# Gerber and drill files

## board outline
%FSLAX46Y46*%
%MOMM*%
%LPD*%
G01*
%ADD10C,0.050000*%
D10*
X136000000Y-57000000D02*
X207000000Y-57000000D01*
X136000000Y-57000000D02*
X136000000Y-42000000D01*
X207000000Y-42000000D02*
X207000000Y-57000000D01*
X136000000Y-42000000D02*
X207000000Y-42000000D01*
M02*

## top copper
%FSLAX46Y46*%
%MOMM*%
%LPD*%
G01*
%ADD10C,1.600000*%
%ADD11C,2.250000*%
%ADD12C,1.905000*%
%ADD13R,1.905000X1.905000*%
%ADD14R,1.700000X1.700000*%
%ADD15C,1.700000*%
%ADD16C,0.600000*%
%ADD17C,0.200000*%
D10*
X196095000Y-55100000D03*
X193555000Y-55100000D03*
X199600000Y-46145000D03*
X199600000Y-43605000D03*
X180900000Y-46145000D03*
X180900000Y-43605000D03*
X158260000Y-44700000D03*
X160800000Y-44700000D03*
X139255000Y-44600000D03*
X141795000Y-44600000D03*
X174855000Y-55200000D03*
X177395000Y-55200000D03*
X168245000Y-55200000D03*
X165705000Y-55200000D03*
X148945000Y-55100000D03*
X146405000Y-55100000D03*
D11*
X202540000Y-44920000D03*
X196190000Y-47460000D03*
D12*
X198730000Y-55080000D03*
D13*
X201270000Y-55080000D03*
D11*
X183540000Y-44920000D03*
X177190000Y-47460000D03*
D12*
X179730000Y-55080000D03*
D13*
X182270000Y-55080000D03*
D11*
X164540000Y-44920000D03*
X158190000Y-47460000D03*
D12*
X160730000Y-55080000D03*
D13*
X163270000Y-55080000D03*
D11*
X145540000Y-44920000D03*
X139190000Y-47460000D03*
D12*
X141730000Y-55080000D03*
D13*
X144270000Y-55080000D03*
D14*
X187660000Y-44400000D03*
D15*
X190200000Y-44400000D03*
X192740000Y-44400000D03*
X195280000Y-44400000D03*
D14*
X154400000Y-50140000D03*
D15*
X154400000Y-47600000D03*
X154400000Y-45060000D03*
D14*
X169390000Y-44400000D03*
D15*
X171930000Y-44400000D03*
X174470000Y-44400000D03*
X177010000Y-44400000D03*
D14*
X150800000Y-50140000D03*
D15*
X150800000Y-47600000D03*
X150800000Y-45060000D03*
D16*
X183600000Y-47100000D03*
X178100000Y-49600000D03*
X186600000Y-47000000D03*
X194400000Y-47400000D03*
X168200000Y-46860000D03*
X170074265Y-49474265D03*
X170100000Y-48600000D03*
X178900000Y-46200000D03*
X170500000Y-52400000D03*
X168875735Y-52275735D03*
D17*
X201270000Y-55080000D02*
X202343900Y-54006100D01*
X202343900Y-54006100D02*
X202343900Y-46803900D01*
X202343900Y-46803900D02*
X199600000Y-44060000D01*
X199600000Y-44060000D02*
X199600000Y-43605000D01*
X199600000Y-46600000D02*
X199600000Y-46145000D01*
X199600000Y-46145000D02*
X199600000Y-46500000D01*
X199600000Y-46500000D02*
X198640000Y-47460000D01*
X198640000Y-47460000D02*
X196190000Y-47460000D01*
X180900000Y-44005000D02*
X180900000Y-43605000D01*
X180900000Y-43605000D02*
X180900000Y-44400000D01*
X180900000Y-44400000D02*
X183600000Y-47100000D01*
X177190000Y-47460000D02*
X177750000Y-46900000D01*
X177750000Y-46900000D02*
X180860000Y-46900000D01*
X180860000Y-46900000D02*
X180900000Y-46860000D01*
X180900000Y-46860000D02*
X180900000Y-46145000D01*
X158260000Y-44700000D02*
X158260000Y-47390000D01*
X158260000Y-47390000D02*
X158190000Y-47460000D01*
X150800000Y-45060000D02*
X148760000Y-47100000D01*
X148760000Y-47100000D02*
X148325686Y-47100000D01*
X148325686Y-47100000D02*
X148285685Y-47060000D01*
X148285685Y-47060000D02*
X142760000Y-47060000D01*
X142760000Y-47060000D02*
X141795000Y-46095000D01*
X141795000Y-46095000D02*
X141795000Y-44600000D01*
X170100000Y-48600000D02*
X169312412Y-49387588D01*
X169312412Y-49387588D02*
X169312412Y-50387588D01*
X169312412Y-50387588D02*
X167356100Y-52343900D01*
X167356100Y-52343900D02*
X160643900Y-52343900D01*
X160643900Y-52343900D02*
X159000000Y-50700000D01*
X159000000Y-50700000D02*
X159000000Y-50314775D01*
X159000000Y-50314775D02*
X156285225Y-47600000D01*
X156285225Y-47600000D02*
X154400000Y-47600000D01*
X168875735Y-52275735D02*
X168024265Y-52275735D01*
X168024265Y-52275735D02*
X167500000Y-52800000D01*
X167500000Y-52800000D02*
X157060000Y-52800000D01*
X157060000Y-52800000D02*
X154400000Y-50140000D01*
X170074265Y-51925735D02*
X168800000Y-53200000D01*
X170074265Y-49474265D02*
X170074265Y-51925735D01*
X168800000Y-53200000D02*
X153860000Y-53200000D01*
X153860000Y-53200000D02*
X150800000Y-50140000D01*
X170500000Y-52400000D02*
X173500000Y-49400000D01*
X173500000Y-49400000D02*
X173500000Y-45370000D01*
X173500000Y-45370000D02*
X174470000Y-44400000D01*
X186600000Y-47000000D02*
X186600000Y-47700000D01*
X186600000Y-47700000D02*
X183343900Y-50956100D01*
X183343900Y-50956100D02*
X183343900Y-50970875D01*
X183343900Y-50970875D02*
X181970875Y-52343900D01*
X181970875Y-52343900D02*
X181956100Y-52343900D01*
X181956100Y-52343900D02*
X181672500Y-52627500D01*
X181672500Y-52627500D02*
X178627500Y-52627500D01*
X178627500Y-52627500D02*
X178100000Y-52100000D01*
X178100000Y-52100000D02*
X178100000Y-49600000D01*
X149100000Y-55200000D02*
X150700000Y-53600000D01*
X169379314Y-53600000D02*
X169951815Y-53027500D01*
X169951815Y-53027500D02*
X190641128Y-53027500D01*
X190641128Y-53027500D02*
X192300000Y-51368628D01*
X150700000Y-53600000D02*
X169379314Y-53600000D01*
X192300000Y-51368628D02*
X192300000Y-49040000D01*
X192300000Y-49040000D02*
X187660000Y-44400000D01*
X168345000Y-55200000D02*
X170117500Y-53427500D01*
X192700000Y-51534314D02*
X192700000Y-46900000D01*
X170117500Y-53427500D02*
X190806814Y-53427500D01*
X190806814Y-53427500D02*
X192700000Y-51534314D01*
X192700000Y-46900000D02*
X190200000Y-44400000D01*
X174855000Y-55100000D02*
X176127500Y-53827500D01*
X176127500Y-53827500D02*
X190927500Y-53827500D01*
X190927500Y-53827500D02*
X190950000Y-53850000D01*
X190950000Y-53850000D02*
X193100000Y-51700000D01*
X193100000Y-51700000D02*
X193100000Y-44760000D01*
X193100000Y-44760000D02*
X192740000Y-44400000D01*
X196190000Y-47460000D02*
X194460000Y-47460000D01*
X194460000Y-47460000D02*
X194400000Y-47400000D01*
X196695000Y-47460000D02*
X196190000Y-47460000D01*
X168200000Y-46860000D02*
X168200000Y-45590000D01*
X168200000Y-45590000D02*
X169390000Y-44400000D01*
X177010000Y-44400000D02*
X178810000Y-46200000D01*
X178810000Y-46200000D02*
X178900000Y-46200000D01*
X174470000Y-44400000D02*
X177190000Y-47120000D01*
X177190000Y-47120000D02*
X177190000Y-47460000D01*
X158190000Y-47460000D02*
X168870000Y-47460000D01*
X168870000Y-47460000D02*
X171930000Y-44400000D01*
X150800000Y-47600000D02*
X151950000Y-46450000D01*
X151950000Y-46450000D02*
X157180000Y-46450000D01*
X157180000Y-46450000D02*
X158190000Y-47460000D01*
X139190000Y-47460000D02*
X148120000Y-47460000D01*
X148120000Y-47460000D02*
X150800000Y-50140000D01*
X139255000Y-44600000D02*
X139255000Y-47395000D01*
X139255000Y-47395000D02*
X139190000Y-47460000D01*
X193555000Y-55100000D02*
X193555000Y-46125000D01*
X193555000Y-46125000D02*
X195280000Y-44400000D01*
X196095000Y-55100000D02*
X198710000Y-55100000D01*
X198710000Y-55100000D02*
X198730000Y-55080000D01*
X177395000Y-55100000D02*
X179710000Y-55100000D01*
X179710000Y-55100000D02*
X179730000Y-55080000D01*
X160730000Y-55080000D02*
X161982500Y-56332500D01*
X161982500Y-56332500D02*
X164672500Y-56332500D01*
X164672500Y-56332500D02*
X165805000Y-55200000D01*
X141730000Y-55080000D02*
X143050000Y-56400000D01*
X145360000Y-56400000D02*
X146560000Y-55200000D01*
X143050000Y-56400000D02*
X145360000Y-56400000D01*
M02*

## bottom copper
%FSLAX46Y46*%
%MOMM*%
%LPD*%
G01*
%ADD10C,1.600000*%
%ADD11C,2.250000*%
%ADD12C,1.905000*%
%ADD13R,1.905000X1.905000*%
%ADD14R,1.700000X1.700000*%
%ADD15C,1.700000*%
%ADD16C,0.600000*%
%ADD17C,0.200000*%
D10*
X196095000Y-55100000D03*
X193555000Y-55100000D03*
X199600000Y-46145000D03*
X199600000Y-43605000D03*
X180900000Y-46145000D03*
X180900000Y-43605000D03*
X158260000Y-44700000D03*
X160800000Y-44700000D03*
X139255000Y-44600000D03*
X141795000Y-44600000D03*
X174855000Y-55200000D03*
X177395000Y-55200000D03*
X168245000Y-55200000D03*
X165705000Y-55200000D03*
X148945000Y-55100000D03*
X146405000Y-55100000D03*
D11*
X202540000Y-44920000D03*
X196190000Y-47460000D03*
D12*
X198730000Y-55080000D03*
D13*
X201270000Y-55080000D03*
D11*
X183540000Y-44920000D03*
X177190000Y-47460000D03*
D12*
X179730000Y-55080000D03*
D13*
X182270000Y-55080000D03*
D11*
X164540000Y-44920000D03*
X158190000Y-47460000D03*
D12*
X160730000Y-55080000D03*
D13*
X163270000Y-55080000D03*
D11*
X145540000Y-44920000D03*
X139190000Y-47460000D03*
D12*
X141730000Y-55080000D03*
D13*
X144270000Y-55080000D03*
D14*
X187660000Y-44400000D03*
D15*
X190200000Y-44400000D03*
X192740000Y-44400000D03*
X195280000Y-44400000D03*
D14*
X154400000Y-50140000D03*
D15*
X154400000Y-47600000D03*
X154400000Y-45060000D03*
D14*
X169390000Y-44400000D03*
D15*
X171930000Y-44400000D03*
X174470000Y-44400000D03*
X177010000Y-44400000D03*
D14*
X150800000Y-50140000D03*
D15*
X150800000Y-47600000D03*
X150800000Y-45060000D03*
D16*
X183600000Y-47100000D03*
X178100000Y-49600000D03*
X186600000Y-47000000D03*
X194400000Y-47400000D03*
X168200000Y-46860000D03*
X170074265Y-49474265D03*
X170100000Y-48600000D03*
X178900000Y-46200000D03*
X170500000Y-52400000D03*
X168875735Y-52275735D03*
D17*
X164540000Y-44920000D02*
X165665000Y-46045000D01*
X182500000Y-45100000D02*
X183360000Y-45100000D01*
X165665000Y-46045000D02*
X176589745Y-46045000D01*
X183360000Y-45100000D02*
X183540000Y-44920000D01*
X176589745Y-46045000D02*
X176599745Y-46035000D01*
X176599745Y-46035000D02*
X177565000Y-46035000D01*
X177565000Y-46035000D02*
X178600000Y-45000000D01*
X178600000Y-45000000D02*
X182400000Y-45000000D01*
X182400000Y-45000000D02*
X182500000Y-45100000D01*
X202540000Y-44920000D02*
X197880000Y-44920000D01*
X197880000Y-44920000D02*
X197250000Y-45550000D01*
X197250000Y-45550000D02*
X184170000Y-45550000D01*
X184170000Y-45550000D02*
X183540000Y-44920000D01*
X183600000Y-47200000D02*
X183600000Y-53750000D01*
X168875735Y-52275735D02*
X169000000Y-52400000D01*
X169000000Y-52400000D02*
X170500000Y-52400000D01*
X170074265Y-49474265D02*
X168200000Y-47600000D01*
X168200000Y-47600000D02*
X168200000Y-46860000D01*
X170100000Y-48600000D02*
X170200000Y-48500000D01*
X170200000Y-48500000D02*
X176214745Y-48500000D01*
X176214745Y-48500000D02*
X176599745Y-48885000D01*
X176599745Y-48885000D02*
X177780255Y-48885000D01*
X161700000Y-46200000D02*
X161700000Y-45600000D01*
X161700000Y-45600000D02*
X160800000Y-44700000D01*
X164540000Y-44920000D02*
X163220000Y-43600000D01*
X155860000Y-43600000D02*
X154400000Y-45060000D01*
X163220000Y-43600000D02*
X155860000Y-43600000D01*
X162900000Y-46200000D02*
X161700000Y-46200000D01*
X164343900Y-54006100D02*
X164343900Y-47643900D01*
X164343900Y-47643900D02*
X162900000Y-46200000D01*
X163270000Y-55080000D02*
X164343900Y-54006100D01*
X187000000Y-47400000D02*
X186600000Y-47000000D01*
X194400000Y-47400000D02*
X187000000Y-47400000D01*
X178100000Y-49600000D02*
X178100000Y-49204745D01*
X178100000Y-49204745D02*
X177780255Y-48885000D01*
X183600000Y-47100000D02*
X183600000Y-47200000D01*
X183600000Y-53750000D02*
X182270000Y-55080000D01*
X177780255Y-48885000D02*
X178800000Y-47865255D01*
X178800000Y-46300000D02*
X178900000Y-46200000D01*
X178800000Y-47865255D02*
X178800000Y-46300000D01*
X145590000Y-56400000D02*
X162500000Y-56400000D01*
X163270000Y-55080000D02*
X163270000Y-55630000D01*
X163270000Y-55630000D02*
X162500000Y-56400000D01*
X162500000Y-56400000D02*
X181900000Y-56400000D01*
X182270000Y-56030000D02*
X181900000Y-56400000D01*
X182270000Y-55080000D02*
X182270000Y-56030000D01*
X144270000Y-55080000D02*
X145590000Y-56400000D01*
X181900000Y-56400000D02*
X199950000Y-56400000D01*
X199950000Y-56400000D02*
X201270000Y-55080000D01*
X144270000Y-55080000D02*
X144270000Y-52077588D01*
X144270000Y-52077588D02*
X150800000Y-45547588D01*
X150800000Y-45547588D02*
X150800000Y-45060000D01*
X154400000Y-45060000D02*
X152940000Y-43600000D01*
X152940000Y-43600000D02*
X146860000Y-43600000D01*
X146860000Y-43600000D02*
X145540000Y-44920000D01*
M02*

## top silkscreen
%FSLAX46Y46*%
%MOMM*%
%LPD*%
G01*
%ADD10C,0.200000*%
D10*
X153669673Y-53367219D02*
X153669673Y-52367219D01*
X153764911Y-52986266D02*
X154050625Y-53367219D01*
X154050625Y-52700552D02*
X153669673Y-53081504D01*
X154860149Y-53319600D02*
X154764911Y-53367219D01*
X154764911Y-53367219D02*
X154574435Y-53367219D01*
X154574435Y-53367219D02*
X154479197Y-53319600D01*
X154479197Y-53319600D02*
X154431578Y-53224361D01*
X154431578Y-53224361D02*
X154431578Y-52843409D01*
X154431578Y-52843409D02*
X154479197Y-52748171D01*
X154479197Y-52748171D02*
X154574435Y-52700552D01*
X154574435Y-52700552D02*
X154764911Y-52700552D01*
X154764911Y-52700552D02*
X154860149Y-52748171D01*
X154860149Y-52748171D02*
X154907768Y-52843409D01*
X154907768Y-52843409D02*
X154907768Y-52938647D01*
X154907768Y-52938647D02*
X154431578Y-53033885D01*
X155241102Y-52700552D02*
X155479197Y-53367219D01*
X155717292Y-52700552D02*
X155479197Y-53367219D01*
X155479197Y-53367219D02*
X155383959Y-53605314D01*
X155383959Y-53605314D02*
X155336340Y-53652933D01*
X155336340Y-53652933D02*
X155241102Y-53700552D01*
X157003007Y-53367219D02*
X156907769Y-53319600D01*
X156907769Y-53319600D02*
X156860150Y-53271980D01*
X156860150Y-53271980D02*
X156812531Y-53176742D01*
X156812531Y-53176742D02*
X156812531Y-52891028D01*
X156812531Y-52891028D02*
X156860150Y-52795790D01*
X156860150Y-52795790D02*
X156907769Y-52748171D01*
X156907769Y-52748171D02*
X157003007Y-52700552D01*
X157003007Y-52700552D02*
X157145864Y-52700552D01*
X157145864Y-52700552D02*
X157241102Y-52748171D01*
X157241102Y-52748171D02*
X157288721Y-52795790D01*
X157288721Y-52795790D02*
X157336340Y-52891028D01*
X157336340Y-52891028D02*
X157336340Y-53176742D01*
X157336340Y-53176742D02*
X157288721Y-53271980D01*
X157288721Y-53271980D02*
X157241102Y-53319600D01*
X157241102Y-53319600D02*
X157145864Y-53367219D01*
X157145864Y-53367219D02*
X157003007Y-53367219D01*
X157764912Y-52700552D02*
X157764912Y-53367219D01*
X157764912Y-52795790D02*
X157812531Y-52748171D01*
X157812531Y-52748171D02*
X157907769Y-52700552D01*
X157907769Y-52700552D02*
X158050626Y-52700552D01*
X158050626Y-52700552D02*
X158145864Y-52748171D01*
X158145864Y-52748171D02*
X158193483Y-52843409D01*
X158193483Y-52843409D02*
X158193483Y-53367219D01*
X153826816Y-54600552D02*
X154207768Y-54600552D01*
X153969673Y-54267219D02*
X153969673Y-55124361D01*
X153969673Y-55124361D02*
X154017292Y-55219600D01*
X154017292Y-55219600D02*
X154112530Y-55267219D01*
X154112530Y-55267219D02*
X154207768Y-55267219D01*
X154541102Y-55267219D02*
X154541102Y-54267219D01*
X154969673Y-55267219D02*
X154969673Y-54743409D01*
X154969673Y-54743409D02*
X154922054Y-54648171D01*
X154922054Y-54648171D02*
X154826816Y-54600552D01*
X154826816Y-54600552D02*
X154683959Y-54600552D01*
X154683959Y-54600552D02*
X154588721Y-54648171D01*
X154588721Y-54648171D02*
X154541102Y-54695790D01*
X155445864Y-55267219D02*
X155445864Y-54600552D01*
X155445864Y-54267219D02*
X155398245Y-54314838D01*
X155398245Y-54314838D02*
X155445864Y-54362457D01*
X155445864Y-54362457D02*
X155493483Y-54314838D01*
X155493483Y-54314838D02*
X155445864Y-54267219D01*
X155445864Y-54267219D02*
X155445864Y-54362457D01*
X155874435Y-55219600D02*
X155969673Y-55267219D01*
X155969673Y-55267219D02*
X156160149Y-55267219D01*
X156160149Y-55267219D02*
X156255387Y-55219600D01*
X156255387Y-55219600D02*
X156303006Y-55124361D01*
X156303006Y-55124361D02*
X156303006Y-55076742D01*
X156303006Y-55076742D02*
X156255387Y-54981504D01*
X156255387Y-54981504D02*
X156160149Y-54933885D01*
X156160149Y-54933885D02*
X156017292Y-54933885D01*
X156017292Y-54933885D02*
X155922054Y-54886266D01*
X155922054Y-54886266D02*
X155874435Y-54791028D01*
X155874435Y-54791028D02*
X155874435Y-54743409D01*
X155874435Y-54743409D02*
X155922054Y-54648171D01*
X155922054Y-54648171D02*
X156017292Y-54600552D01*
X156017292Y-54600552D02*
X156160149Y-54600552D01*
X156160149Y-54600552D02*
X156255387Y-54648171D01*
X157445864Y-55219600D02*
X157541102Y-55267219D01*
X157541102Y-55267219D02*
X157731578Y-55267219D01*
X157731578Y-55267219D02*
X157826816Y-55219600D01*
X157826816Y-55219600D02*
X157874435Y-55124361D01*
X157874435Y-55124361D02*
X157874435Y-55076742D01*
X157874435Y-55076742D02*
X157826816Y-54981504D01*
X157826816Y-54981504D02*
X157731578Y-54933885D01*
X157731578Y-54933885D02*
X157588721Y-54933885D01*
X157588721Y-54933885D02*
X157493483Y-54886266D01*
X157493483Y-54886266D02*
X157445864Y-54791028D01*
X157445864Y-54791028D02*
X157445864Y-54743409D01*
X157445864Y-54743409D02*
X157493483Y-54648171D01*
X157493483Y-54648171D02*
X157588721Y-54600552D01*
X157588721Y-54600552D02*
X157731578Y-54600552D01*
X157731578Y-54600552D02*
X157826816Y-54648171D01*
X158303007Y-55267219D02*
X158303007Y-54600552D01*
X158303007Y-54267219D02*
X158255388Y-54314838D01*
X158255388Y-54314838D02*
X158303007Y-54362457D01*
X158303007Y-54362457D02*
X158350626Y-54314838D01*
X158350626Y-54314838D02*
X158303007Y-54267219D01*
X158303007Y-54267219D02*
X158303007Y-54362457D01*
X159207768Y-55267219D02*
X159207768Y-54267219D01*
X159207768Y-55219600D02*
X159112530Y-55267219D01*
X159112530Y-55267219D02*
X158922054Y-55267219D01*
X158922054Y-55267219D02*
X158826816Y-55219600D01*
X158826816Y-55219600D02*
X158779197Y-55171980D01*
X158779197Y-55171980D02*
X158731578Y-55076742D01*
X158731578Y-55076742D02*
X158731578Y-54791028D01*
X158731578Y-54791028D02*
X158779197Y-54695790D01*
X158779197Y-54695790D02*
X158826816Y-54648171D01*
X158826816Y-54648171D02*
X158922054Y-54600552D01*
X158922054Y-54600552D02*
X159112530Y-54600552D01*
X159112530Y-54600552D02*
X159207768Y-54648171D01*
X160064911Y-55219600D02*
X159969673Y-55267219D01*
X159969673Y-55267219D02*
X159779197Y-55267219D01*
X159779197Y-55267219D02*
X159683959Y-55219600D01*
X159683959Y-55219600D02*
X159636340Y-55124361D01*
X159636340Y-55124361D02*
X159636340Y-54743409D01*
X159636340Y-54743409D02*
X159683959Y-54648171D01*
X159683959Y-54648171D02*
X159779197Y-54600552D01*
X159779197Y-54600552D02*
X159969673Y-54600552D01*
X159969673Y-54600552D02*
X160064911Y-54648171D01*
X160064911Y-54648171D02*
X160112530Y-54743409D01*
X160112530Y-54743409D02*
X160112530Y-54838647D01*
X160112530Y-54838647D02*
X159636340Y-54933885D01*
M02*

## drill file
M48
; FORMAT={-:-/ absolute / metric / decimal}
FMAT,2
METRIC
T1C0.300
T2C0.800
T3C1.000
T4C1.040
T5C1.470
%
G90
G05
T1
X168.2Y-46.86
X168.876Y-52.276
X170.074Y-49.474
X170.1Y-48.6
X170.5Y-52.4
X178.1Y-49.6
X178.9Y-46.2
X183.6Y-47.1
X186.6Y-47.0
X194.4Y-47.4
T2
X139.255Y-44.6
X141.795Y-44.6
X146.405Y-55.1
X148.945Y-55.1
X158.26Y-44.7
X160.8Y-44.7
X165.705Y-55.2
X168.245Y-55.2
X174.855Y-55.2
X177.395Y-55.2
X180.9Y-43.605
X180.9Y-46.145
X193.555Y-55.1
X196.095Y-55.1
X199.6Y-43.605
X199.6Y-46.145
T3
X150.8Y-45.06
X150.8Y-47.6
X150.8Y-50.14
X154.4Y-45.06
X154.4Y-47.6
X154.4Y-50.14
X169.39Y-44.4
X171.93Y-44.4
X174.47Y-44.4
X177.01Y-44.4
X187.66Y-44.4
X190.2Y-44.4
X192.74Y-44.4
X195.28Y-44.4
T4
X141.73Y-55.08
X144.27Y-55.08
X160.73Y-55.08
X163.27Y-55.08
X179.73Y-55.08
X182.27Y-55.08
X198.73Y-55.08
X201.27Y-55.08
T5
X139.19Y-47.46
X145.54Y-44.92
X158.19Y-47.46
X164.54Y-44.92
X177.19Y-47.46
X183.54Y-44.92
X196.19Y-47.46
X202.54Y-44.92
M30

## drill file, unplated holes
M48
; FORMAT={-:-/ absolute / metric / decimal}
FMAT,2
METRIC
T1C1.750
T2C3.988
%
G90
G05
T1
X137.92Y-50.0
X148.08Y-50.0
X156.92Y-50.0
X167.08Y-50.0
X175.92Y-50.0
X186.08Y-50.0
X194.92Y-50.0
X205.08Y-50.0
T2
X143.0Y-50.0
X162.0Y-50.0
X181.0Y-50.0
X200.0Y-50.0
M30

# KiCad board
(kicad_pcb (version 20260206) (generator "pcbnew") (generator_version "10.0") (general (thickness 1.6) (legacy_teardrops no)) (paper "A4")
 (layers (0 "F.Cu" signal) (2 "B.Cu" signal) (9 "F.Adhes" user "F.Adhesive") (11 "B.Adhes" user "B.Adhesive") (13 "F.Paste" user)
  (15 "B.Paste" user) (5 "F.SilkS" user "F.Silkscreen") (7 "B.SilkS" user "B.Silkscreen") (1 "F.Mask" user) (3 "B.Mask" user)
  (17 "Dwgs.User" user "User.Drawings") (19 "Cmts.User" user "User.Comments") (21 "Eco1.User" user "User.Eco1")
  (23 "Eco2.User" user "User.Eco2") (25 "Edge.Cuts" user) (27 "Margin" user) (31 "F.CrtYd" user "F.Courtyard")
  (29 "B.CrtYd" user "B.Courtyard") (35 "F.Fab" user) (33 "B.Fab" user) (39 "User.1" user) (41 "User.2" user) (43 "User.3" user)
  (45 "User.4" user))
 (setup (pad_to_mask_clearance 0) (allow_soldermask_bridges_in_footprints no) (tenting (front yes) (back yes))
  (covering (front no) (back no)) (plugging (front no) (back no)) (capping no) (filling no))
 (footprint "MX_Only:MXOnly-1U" (layer "F.Cu") (at 200 50)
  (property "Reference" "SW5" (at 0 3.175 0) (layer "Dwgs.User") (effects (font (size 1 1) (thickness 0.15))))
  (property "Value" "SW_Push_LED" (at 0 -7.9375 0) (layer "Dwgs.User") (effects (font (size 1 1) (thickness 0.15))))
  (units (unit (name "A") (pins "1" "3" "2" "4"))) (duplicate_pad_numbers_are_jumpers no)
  (pad "" np_thru_hole circle (at -5.08 0 48.0996) (size 1.75 1.75) (drill 1.75) (layers "*.Cu" "*.Mask"))
  (pad "" np_thru_hole circle (at 0 0) (size 3.9878 3.9878) (drill 3.9878) (layers "*.Cu" "*.Mask"))
  (pad "" np_thru_hole circle (at 5.08 0 48.0996) (size 1.75 1.75) (drill 1.75) (layers "*.Cu" "*.Mask"))
  (pad "1" thru_hole circle (at -3.81 -2.54) (size 2.25 2.25) (drill 1.47) (layers "*.Cu" "B.Mask") (remove_unused_layers no) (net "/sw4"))
  (pad "2" thru_hole circle (at 2.54 -5.08) (size 2.25 2.25) (drill 1.47) (layers "*.Cu" "B.Mask") (remove_unused_layers no) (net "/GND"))
  (pad "3" thru_hole circle (at -1.27 5.08) (size 1.905 1.905) (drill 1.04) (layers "*.Cu" "B.Mask") (remove_unused_layers no)
   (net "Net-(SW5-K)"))
  (pad "4" thru_hole rect (at 1.27 5.08) (size 1.905 1.905) (drill 1.04) (layers "*.Cu" "B.Mask") (remove_unused_layers no) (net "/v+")))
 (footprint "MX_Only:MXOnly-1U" (layer "F.Cu") (at 162 50)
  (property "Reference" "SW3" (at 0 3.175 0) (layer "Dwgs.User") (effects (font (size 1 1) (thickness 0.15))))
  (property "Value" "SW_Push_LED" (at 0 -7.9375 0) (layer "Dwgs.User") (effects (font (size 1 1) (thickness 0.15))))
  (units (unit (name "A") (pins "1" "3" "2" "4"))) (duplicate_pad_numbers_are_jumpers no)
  (pad "" np_thru_hole circle (at -5.08 0 48.0996) (size 1.75 1.75) (drill 1.75) (layers "*.Cu" "*.Mask"))
  (pad "" np_thru_hole circle (at 0 0) (size 3.9878 3.9878) (drill 3.9878) (layers "*.Cu" "*.Mask"))
  (pad "" np_thru_hole circle (at 5.08 0 48.0996) (size 1.75 1.75) (drill 1.75) (layers "*.Cu" "*.Mask"))
  (pad "1" thru_hole circle (at -3.81 -2.54) (size 2.25 2.25) (drill 1.47) (layers "*.Cu" "B.Mask") (remove_unused_layers no) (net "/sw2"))
  (pad "2" thru_hole circle (at 2.54 -5.08) (size 2.25 2.25) (drill 1.47) (layers "*.Cu" "B.Mask") (remove_unused_layers no) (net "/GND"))
  (pad "3" thru_hole circle (at -1.27 5.08) (size 1.905 1.905) (drill 1.04) (layers "*.Cu" "B.Mask") (remove_unused_layers no)
   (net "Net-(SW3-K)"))
  (pad "4" thru_hole rect (at 1.27 5.08) (size 1.905 1.905) (drill 1.04) (layers "*.Cu" "B.Mask") (remove_unused_layers no) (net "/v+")))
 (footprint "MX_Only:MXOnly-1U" (layer "F.Cu") (at 181 50)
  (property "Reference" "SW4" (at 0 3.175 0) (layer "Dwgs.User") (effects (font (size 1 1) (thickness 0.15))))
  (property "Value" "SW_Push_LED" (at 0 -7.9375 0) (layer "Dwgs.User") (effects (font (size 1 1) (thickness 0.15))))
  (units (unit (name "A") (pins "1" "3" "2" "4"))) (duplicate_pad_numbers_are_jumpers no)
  (pad "" np_thru_hole circle (at -5.08 0 48.0996) (size 1.75 1.75) (drill 1.75) (layers "*.Cu" "*.Mask"))
  (pad "" np_thru_hole circle (at 0 0) (size 3.9878 3.9878) (drill 3.9878) (layers "*.Cu" "*.Mask"))
  (pad "" np_thru_hole circle (at 5.08 0 48.0996) (size 1.75 1.75) (drill 1.75) (layers "*.Cu" "*.Mask"))
  (pad "1" thru_hole circle (at -3.81 -2.54) (size 2.25 2.25) (drill 1.47) (layers "*.Cu" "B.Mask") (remove_unused_layers no) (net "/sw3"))
  (pad "2" thru_hole circle (at 2.54 -5.08) (size 2.25 2.25) (drill 1.47) (layers "*.Cu" "B.Mask") (remove_unused_layers no) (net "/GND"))
  (pad "3" thru_hole circle (at -1.27 5.08) (size 1.905 1.905) (drill 1.04) (layers "*.Cu" "B.Mask") (remove_unused_layers no)
   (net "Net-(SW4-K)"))
  (pad "4" thru_hole rect (at 1.27 5.08) (size 1.905 1.905) (drill 1.04) (layers "*.Cu" "B.Mask") (remove_unused_layers no) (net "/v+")))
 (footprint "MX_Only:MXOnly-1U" (layer "F.Cu") (at 143 50)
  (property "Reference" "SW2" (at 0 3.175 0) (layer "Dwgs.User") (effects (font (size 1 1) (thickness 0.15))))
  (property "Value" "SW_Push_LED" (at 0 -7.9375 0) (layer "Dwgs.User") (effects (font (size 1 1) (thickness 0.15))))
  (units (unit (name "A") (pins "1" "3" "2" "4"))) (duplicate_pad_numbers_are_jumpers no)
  (pad "" np_thru_hole circle (at -5.08 0 48.0996) (size 1.75 1.75) (drill 1.75) (layers "*.Cu" "*.Mask"))
  (pad "" np_thru_hole circle (at 0 0) (size 3.9878 3.9878) (drill 3.9878) (layers "*.Cu" "*.Mask"))
  (pad "" np_thru_hole circle (at 5.08 0 48.0996) (size 1.75 1.75) (drill 1.75) (layers "*.Cu" "*.Mask"))
  (pad "1" thru_hole circle (at -3.81 -2.54) (size 2.25 2.25) (drill 1.47) (layers "*.Cu" "B.Mask") (remove_unused_layers no) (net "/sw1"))
  (pad "2" thru_hole circle (at 2.54 -5.08) (size 2.25 2.25) (drill 1.47) (layers "*.Cu" "B.Mask") (remove_unused_layers no) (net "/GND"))
  (pad "3" thru_hole circle (at -1.27 5.08) (size 1.905 1.905) (drill 1.04) (layers "*.Cu" "B.Mask") (remove_unused_layers no)
   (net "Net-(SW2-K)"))
  (pad "4" thru_hole rect (at 1.27 5.08) (size 1.905 1.905) (drill 1.04) (layers "*.Cu" "B.Mask") (remove_unused_layers no) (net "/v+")))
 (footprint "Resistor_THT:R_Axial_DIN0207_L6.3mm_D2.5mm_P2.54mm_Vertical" (layer "B.Cu") (at 174.855 55.2)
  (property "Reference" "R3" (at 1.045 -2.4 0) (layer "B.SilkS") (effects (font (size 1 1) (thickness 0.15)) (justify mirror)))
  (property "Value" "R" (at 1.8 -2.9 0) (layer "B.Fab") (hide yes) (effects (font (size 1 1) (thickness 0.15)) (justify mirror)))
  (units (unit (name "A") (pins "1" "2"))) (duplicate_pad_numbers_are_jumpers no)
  (pad "1" thru_hole circle (at 0 0) (size 1.6 1.6) (drill 0.8) (layers "*.Cu" "*.Mask") (remove_unused_layers no) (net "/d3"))
  (pad "2" thru_hole circle (at 2.54 0) (size 1.6 1.6) (drill 0.8) (layers "*.Cu" "*.Mask") (remove_unused_layers no) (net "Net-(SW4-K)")))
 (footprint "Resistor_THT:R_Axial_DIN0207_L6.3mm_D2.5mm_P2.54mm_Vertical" (layer "B.Cu") (at 193.555 55.1)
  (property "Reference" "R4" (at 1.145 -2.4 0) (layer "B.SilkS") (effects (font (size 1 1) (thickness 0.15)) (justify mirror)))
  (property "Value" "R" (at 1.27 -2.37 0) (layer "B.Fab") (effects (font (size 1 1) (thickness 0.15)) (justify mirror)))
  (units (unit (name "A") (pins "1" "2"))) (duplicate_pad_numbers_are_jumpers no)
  (pad "1" thru_hole circle (at 0 0) (size 1.6 1.6) (drill 0.8) (layers "*.Cu" "*.Mask") (remove_unused_layers no) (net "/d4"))
  (pad "2" thru_hole circle (at 2.54 0) (size 1.6 1.6) (drill 0.8) (layers "*.Cu" "*.Mask") (remove_unused_layers no) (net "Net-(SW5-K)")))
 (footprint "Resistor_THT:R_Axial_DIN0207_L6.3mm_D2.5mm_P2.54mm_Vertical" (layer "B.Cu") (at 158.26 44.7)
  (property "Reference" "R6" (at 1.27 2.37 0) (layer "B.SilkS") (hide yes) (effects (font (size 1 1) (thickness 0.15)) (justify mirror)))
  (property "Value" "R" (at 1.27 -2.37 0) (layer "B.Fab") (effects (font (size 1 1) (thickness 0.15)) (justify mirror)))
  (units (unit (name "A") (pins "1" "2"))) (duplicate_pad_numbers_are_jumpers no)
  (pad "1" thru_hole circle (at 0 0) (size 1.6 1.6) (drill 0.8) (layers "*.Cu" "*.Mask") (remove_unused_layers no) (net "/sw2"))
  (pad "2" thru_hole circle (at 2.54 0) (size 1.6 1.6) (drill 0.8) (layers "*.Cu" "*.Mask") (remove_unused_layers no) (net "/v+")))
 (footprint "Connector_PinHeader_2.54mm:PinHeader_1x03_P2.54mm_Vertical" (layer "B.Cu") (at 154.4 50.14)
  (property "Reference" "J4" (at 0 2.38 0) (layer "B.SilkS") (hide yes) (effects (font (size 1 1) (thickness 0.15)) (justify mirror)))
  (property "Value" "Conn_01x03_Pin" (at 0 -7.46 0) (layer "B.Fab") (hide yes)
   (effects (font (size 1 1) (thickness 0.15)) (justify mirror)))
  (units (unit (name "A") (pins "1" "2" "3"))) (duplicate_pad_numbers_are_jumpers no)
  (pad "1" thru_hole rect (at 0 0) (size 1.7 1.7) (drill 1) (layers "*.Cu" "*.Mask") (remove_unused_layers no) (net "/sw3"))
  (pad "2" thru_hole circle (at 0 -2.54) (size 1.7 1.7) (drill 1) (layers "*.Cu" "*.Mask") (remove_unused_layers no) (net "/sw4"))
  (pad "3" thru_hole circle (at 0 -5.08) (size 1.7 1.7) (drill 1) (layers "*.Cu" "*.Mask") (remove_unused_layers no) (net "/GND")))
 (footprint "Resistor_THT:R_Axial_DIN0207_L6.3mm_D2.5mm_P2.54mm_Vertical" (layer "B.Cu") (at 168.245 55.2 180)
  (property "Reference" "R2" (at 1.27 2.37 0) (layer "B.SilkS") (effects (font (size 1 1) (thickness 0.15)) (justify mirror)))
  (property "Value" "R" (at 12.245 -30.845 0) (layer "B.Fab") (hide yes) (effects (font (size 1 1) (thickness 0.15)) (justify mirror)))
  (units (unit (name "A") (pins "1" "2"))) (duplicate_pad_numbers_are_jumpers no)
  (pad "1" thru_hole circle (at 0 0 180) (size 1.6 1.6) (drill 0.8) (layers "*.Cu" "*.Mask") (remove_unused_layers no) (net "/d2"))
  (pad "2" thru_hole circle (at 2.54 0 180) (size 1.6 1.6) (drill 0.8) (layers "*.Cu" "*.Mask") (remove_unused_layers no)
   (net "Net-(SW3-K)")))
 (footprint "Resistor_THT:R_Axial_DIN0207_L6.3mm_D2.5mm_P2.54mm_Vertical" (layer "B.Cu") (at 180.9 46.145 90)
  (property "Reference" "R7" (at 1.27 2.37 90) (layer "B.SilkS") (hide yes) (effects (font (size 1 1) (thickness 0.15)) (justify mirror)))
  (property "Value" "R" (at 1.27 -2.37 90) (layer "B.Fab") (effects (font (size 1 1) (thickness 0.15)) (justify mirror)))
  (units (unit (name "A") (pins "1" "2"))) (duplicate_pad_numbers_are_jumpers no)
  (pad "1" thru_hole circle (at 0 0 90) (size 1.6 1.6) (drill 0.8) (layers "*.Cu" "*.Mask") (remove_unused_layers no) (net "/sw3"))
  (pad "2" thru_hole circle (at 2.54 0 90) (size 1.6 1.6) (drill 0.8) (layers "*.Cu" "*.Mask") (remove_unused_layers no) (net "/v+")))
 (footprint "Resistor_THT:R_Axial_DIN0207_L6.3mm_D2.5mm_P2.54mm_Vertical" (layer "B.Cu") (at 148.945 55.1 180)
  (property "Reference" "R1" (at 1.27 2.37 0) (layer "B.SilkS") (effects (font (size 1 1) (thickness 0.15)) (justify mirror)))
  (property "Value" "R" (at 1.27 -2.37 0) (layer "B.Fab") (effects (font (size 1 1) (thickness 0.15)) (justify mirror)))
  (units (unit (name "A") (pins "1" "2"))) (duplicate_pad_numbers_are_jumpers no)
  (pad "1" thru_hole circle (at 0 0 180) (size 1.6 1.6) (drill 0.8) (layers "*.Cu" "*.Mask") (remove_unused_layers no) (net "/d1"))
  (pad "2" thru_hole circle (at 2.54 0 180) (size 1.6 1.6) (drill 0.8) (layers "*.Cu" "*.Mask") (remove_unused_layers no)
   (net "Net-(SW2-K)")))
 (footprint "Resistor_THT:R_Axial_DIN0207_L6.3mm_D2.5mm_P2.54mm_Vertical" (layer "B.Cu") (at 139.255 44.6)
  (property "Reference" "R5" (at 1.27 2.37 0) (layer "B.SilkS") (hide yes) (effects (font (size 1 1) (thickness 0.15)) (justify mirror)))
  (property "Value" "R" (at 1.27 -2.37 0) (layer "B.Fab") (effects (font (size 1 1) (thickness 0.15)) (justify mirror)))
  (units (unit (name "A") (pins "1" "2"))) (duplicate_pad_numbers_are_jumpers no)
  (pad "1" thru_hole circle (at 0 0) (size 1.6 1.6) (drill 0.8) (layers "*.Cu" "*.Mask") (remove_unused_layers no) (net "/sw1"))
  (pad "2" thru_hole circle (at 2.54 0) (size 1.6 1.6) (drill 0.8) (layers "*.Cu" "*.Mask") (remove_unused_layers no) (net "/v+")))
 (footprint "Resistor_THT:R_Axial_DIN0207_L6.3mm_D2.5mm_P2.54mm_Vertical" (layer "B.Cu") (at 199.6 46.145 90)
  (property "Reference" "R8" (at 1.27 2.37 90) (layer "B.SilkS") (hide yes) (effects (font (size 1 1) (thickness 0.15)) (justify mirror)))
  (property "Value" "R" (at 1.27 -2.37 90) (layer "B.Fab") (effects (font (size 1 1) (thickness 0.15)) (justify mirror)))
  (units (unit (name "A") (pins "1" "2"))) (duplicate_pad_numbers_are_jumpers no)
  (pad "1" thru_hole circle (at 0 0 90) (size 1.6 1.6) (drill 0.8) (layers "*.Cu" "*.Mask") (remove_unused_layers no) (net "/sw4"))
  (pad "2" thru_hole circle (at 2.54 0 90) (size 1.6 1.6) (drill 0.8) (layers "*.Cu" "*.Mask") (remove_unused_layers no) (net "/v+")))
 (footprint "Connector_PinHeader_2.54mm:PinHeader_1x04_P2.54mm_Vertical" (layer "B.Cu") (at 169.39 44.4 -90)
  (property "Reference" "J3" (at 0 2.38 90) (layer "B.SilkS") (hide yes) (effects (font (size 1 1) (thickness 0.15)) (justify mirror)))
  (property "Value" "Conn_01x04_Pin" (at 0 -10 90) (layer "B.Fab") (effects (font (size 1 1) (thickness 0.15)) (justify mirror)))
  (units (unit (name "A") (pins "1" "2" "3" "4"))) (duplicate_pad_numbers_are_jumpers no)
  (pad "1" thru_hole rect (at 0 0 270) (size 1.7 1.7) (drill 1) (layers "*.Cu" "*.Mask") (remove_unused_layers no) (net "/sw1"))
  (pad "2" thru_hole circle (at 0 -2.54 270) (size 1.7 1.7) (drill 1) (layers "*.Cu" "*.Mask") (remove_unused_layers no) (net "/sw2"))
  (pad "3" thru_hole circle (at 0 -5.08 270) (size 1.7 1.7) (drill 1) (layers "*.Cu" "*.Mask") (remove_unused_layers no) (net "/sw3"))
  (pad "4" thru_hole circle (at 0 -7.62 270) (size 1.7 1.7) (drill 1) (layers "*.Cu" "*.Mask") (remove_unused_layers no) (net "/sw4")))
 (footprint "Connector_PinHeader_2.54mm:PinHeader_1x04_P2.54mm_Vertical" (layer "B.Cu") (at 187.66 44.4 -90)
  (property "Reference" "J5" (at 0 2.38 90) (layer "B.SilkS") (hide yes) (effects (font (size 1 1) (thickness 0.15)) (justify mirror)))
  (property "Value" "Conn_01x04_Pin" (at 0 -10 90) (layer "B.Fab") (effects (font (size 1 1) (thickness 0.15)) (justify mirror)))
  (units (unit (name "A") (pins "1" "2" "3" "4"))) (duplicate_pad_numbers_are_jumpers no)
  (pad "1" thru_hole rect (at 0 0 270) (size 1.7 1.7) (drill 1) (layers "*.Cu" "*.Mask") (remove_unused_layers no) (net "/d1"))
  (pad "2" thru_hole circle (at 0 -2.54 270) (size 1.7 1.7) (drill 1) (layers "*.Cu" "*.Mask") (remove_unused_layers no) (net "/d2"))
  (pad "3" thru_hole circle (at 0 -5.08 270) (size 1.7 1.7) (drill 1) (layers "*.Cu" "*.Mask") (remove_unused_layers no) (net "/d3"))
  (pad "4" thru_hole circle (at 0 -7.62 270) (size 1.7 1.7) (drill 1) (layers "*.Cu" "*.Mask") (remove_unused_layers no) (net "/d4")))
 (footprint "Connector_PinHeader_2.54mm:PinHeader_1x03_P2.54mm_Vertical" (layer "B.Cu") (at 150.8 50.14)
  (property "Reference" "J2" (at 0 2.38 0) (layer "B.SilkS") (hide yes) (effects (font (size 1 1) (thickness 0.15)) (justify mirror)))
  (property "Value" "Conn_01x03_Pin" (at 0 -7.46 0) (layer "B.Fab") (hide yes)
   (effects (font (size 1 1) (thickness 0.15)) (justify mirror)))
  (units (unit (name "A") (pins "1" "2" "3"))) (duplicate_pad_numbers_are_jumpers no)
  (pad "1" thru_hole rect (at 0 0) (size 1.7 1.7) (drill 1) (layers "*.Cu" "*.Mask") (remove_unused_layers no) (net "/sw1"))
  (pad "2" thru_hole circle (at 0 -2.54) (size 1.7 1.7) (drill 1) (layers "*.Cu" "*.Mask") (remove_unused_layers no) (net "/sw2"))
  (pad "3" thru_hole circle (at 0 -5.08) (size 1.7 1.7) (drill 1) (layers "*.Cu" "*.Mask") (remove_unused_layers no) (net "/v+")))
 (gr_line (start 136 42) (end 207 42) (stroke (width 0.05) (type solid)) (layer "Edge.Cuts"))
 (gr_line (start 136 57) (end 136 42) (stroke (width 0.05) (type default)) (layer "Edge.Cuts"))
 (gr_line (start 136 57) (end 207 57) (stroke (width 0.05) (type solid)) (layer "Edge.Cuts"))
 (gr_line (start 207 42) (end 207 57) (stroke (width 0.05) (type solid)) (layer "Edge.Cuts"))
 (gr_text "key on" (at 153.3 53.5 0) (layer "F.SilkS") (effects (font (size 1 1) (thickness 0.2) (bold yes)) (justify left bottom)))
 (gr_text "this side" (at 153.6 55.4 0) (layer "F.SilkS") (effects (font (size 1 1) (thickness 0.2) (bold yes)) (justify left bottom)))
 (segment (start 199.6 44.06) (end 199.6 43.605) (width 0.2) (layer "F.Cu") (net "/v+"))
 (segment (start 201.27 55.08) (end 202.3439 54.0061) (width 0.2) (layer "F.Cu") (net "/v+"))
 (segment (start 150.8 45.06) (end 148.76 47.1) (width 0.2) (layer "F.Cu") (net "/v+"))
 (segment (start 180.9 44.005) (end 180.9 43.605) (width 0.2) (layer "F.Cu") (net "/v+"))
 (segment (start 148.76 47.1) (end 148.325686 47.1) (width 0.2) (layer "F.Cu") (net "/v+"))
 (segment (start 142.76 47.06) (end 141.795 46.095) (width 0.2) (layer "F.Cu") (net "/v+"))
 (segment (start 148.325686 47.1) (end 148.285685 47.06) (width 0.2) (layer "F.Cu") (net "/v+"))
 (segment (start 202.3439 54.0061) (end 202.3439 46.8039) (width 0.2) (layer "F.Cu") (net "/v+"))
 (segment (start 180.9 44.4) (end 183.6 47.1) (width 0.2) (layer "F.Cu") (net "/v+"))
 (segment (start 141.795 46.095) (end 141.795 44.6) (width 0.2) (layer "F.Cu") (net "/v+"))
 (segment (start 148.285685 47.06) (end 142.76 47.06) (width 0.2) (layer "F.Cu") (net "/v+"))
 (segment (start 180.9 43.605) (end 180.9 44.4) (width 0.2) (layer "F.Cu") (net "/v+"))
 (segment (start 202.3439 46.8039) (end 199.6 44.06) (width 0.2) (layer "F.Cu") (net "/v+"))
 (via (at 183.6 47.1) (size 0.6) (drill 0.3) (layers "F.Cu" "B.Cu") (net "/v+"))
 (segment (start 163.27 55.63) (end 162.5 56.4) (width 0.2) (layer "B.Cu") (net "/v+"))
 (segment (start 163.27 55.08) (end 164.3439 54.0061) (width 0.2) (layer "B.Cu") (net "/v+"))
 (segment (start 144.27 52.077588) (end 150.8 45.547588) (width 0.2) (layer "B.Cu") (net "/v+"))
 (segment (start 150.8 45.547588) (end 150.8 45.06) (width 0.2) (layer "B.Cu") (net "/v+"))
 (segment (start 161.7 45.6) (end 160.8 44.7) (width 0.2) (layer "B.Cu") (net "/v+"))
 (segment (start 199.95 56.4) (end 201.27 55.08) (width 0.2) (layer "B.Cu") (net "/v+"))
 (segment (start 161.7 46.2) (end 161.7 45.6) (width 0.2) (layer "B.Cu") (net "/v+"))
 (segment (start 183.6 53.75) (end 182.27 55.08) (width 0.2) (layer "B.Cu") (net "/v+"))
 (segment (start 182.27 55.08) (end 182.27 56.03) (width 0.2) (layer "B.Cu") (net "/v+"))
 (segment (start 183.6 47.2) (end 183.6 53.75) (width 0.2) (layer "B.Cu") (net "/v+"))
 (segment (start 144.27 55.08) (end 144.27 52.077588) (width 0.2) (layer "B.Cu") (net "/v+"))
 (segment (start 163.27 55.08) (end 163.27 55.63) (width 0.2) (layer "B.Cu") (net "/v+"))
 (segment (start 144.27 55.08) (end 145.59 56.4) (width 0.2) (layer "B.Cu") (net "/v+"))
 (segment (start 181.9 56.4) (end 199.95 56.4) (width 0.2) (layer "B.Cu") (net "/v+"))
 (segment (start 164.3439 54.0061) (end 164.3439 47.6439) (width 0.2) (layer "B.Cu") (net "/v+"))
 (segment (start 162.9 46.2) (end 161.7 46.2) (width 0.2) (layer "B.Cu") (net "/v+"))
 (segment (start 182.27 56.03) (end 181.9 56.4) (width 0.2) (layer "B.Cu") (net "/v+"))
 (segment (start 164.3439 47.6439) (end 162.9 46.2) (width 0.2) (layer "B.Cu") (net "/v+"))
 (segment (start 162.5 56.4) (end 181.9 56.4) (width 0.2) (layer "B.Cu") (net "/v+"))
 (segment (start 145.59 56.4) (end 162.5 56.4) (width 0.2) (layer "B.Cu") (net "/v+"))
 (segment (start 183.6 47.1) (end 183.6 47.2) (width 0.2) (layer "B.Cu") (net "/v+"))
 (segment (start 149.1 55.2) (end 150.7 53.6) (width 0.2) (layer "F.Cu") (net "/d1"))
 (segment (start 192.3 51.368628) (end 192.3 49.04) (width 0.2) (layer "F.Cu") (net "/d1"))
 (segment (start 192.3 49.04) (end 187.66 44.4) (width 0.2) (layer "F.Cu") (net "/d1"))
 (segment (start 169.951815 53.0275) (end 190.641128 53.0275) (width 0.2) (layer "F.Cu") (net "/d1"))
 (segment (start 190.641128 53.0275) (end 192.3 51.368628) (width 0.2) (layer "F.Cu") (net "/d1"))
 (segment (start 150.7 53.6) (end 169.379314 53.6) (width 0.2) (layer "F.Cu") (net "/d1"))
 (segment (start 169.379314 53.6) (end 169.951815 53.0275) (width 0.2) (layer "F.Cu") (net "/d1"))
 (segment (start 192.7 51.534314) (end 192.7 46.9) (width 0.2) (layer "F.Cu") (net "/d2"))
 (segment (start 170.1175 53.4275) (end 190.806814 53.4275) (width 0.2) (layer "F.Cu") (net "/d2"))
 (segment (start 192.7 46.9) (end 190.2 44.4) (width 0.2) (layer "F.Cu") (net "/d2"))
 (segment (start 190.806814 53.4275) (end 192.7 51.534314) (width 0.2) (layer "F.Cu") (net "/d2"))
 (segment (start 168.345 55.2) (end 170.1175 53.4275) (width 0.2) (layer "F.Cu") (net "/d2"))
 (segment (start 153.86 53.2) (end 150.8 50.14) (width 0.2) (layer "F.Cu") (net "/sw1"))
 (segment (start 168.2 45.59) (end 169.39 44.4) (width 0.2) (layer "F.Cu") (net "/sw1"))
 (segment (start 139.19 47.46) (end 148.12 47.46) (width 0.2) (layer "F.Cu") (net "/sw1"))
 (segment (start 170.074265 51.925735) (end 168.8 53.2) (width 0.2) (layer "F.Cu") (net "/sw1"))
 (segment (start 139.255 47.395) (end 139.19 47.46) (width 0.2) (layer "F.Cu") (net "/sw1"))
 (segment (start 168.2 46.86) (end 168.2 45.59) (width 0.2) (layer "F.Cu") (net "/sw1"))
 (segment (start 139.255 44.6) (end 139.255 47.395) (width 0.2) (layer "F.Cu") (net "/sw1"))
 (segment (start 170.074265 49.474265) (end 170.074265 51.925735) (width 0.2) (layer "F.Cu") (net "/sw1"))
 (segment (start 168.8 53.2) (end 153.86 53.2) (width 0.2) (layer "F.Cu") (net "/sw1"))
 (segment (start 148.12 47.46) (end 150.8 50.14) (width 0.2) (layer "F.Cu") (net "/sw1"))
 (via (at 168.2 46.86) (size 0.6) (drill 0.3) (layers "F.Cu" "B.Cu") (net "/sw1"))
 (via (at 170.074265 49.474265) (size 0.6) (drill 0.3) (layers "F.Cu" "B.Cu") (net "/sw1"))
 (segment (start 168.2 47.6) (end 168.2 46.86) (width 0.2) (layer "B.Cu") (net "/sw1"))
 (segment (start 170.074265 49.474265) (end 168.2 47.6) (width 0.2) (layer "B.Cu") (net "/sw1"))
 (segment (start 193.555 55.1) (end 193.555 46.125) (width 0.2) (layer "F.Cu") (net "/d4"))
 (segment (start 193.555 46.125) (end 195.28 44.4) (width 0.2) (layer "F.Cu") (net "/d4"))
 (segment (start 190.95 53.85) (end 193.1 51.7) (width 0.2) (layer "F.Cu") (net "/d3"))
 (segment (start 193.1 51.7) (end 193.1 44.76) (width 0.2) (layer "F.Cu") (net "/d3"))
 (segment (start 174.855 55.1) (end 176.1275 53.8275) (width 0.2) (layer "F.Cu") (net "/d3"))
 (segment (start 176.1275 53.8275) (end 190.9275 53.8275) (width 0.2) (layer "F.Cu") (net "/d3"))
 (segment (start 190.9275 53.8275) (end 190.95 53.85) (width 0.2) (layer "F.Cu") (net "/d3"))
 (segment (start 193.1 44.76) (end 192.74 44.4) (width 0.2) (layer "F.Cu") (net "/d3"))
 (segment (start 182.5 45.1) (end 183.36 45.1) (width 0.2) (layer "B.Cu") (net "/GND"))
 (segment (start 183.36 45.1) (end 183.54 44.92) (width 0.2) (layer "B.Cu") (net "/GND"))
 (segment (start 163.22 43.6) (end 155.86 43.6) (width 0.2) (layer "B.Cu") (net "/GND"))
 (segment (start 165.665 46.045) (end 176.589745 46.045) (width 0.2) (layer "B.Cu") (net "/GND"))
 (segment (start 197.25 45.55) (end 184.17 45.55) (width 0.2) (layer "B.Cu") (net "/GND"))
 (segment (start 184.17 45.55) (end 183.54 44.92) (width 0.2) (layer "B.Cu") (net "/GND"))
 (segment (start 178.6 45) (end 182.4 45) (width 0.2) (layer "B.Cu") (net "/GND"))
 (segment (start 146.86 43.6) (end 145.54 44.92) (width 0.2) (layer "B.Cu") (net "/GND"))
 (segment (start 154.4 45.06) (end 152.94 43.6) (width 0.2) (layer "B.Cu") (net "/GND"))
 (segment (start 177.565 46.035) (end 178.6 45) (width 0.2) (layer "B.Cu") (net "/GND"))
 (segment (start 164.54 44.92) (end 165.665 46.045) (width 0.2) (layer "B.Cu") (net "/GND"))
 (segment (start 176.589745 46.045) (end 176.599745 46.035) (width 0.2) (layer "B.Cu") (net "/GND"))
 (segment (start 164.54 44.92) (end 163.22 43.6) (width 0.2) (layer "B.Cu") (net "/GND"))
 (segment (start 202.54 44.92) (end 197.88 44.92) (width 0.2) (layer "B.Cu") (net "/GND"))
 (segment (start 155.86 43.6) (end 154.4 45.06) (width 0.2) (layer "B.Cu") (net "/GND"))
 (segment (start 152.94 43.6) (end 146.86 43.6) (width 0.2) (layer "B.Cu") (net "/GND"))
 (segment (start 182.4 45) (end 182.5 45.1) (width 0.2) (layer "B.Cu") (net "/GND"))
 (segment (start 197.88 44.92) (end 197.25 45.55) (width 0.2) (layer "B.Cu") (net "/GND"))
 (segment (start 176.599745 46.035) (end 177.565 46.035) (width 0.2) (layer "B.Cu") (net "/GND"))
 (segment (start 143.05 56.4) (end 145.36 56.4) (width 0.2) (layer "F.Cu") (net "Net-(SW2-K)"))
 (segment (start 145.36 56.4) (end 146.56 55.2) (width 0.2) (layer "F.Cu") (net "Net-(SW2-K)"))
 (segment (start 141.73 55.08) (end 143.05 56.4) (width 0.2) (layer "F.Cu") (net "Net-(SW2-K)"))
 (segment (start 164.6725 56.3325) (end 165.805 55.2) (width 0.2) (layer "F.Cu") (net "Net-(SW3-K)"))
 (segment (start 161.9825 56.3325) (end 164.6725 56.3325) (width 0.2) (layer "F.Cu") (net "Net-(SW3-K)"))
 (segment (start 160.73 55.08) (end 161.9825 56.3325) (width 0.2) (layer "F.Cu") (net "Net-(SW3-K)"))
 (segment (start 179.71 55.1) (end 179.73 55.08) (width 0.2) (layer "F.Cu") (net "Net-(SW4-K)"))
 (segment (start 177.395 55.1) (end 179.71 55.1) (width 0.2) (layer "F.Cu") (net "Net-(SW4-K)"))
 (segment (start 198.71 55.1) (end 198.73 55.08) (width 0.2) (layer "F.Cu") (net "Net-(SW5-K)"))
 (segment (start 196.095 55.1) (end 198.71 55.1) (width 0.2) (layer "F.Cu") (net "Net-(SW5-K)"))
 (segment (start 157.18 46.45) (end 158.19 47.46) (width 0.2) (layer "F.Cu") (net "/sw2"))
 (segment (start 158.19 47.46) (end 168.87 47.46) (width 0.2) (layer "F.Cu") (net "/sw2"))
 (segment (start 150.8 47.6) (end 151.95 46.45) (width 0.2) (layer "F.Cu") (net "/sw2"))
 (segment (start 168.87 47.46) (end 171.93 44.4) (width 0.2) (layer "F.Cu") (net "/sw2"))
 (segment (start 151.95 46.45) (end 157.18 46.45) (width 0.2) (layer "F.Cu") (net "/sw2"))
 (segment (start 158.26 47.39) (end 158.19 47.46) (width 0.2) (layer "F.Cu") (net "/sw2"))
 (segment (start 158.26 44.7) (end 158.26 47.39) (width 0.2) (layer "F.Cu") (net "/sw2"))
 (segment (start 170.5 52.4) (end 173.5 49.4) (width 0.2) (layer "F.Cu") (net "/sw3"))
 (segment (start 177.19 47.12) (end 177.19 47.46) (width 0.2) (layer "F.Cu") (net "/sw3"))
 (segment (start 167.5 52.8) (end 157.06 52.8) (width 0.2) (layer "F.Cu") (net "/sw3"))
 (segment (start 168.024265 52.275735) (end 167.5 52.8) (width 0.2) (layer "F.Cu") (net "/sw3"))
 (segment (start 177.19 47.46) (end 177.75 46.9) (width 0.2) (layer "F.Cu") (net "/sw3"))
 (segment (start 174.47 44.4) (end 177.19 47.12) (width 0.2) (layer "F.Cu") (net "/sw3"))
 (segment (start 173.5 49.4) (end 173.5 45.37) (width 0.2) (layer "F.Cu") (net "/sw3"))
 (segment (start 168.875735 52.275735) (end 168.024265 52.275735) (width 0.2) (layer "F.Cu") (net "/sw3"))
 (segment (start 180.86 46.9) (end 180.9 46.86) (width 0.2) (layer "F.Cu") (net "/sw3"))
 (segment (start 157.06 52.8) (end 154.4 50.14) (width 0.2) (layer "F.Cu") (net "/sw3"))
 (segment (start 173.5 45.37) (end 174.47 44.4) (width 0.2) (layer "F.Cu") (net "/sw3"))
 (segment (start 180.9 46.86) (end 180.9 46.145) (width 0.2) (layer "F.Cu") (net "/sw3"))
 (segment (start 177.75 46.9) (end 180.86 46.9) (width 0.2) (layer "F.Cu") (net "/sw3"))
 (via (at 168.875735 52.275735) (size 0.6) (drill 0.3) (layers "F.Cu" "B.Cu") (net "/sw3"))
 (via (at 170.5 52.4) (size 0.6) (drill 0.3) (layers "F.Cu" "B.Cu") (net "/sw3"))
 (segment (start 168.875735 52.275735) (end 169 52.4) (width 0.2) (layer "B.Cu") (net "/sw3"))
 (segment (start 169 52.4) (end 170.5 52.4) (width 0.2) (layer "B.Cu") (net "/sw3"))
 (segment (start 199.6 46.5) (end 198.64 47.46) (width 0.2) (layer "F.Cu") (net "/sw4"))
 (segment (start 199.6 46.145) (end 199.6 46.5) (width 0.2) (layer "F.Cu") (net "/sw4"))
 (segment (start 159 50.7) (end 159 50.314775) (width 0.2) (layer "F.Cu") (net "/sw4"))
 (segment (start 183.3439 50.9561) (end 183.3439 50.970875) (width 0.2) (layer "F.Cu") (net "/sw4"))
 (segment (start 196.695 47.46) (end 196.19 47.46) (width 0.2) (layer "F.Cu") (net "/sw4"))
 (segment (start 159 50.314775) (end 156.285225 47.6) (width 0.2) (layer "F.Cu") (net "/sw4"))
 (segment (start 181.970875 52.3439) (end 181.9561 52.3439) (width 0.2) (layer "F.Cu") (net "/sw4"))
 (segment (start 160.6439 52.3439) (end 159 50.7) (width 0.2) (layer "F.Cu") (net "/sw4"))
 (segment (start 178.1 52.1) (end 178.1 49.6) (width 0.2) (layer "F.Cu") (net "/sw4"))
 (segment (start 178.81 46.2) (end 178.9 46.2) (width 0.2) (layer "F.Cu") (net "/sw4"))
 (segment (start 183.3439 50.970875) (end 181.970875 52.3439) (width 0.2) (layer "F.Cu") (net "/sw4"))
 (segment (start 156.285225 47.6) (end 154.4 47.6) (width 0.2) (layer "F.Cu") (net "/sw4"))
 (segment (start 198.64 47.46) (end 196.19 47.46) (width 0.2) (layer "F.Cu") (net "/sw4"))
 (segment (start 199.6 46.6) (end 199.6 46.145) (width 0.2) (layer "F.Cu") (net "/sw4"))
 (segment (start 169.312412 49.387588) (end 169.312412 50.387588) (width 0.2) (layer "F.Cu") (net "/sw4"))
 (segment (start 170.1 48.6) (end 169.312412 49.387588) (width 0.2) (layer "F.Cu") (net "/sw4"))
 (segment (start 167.3561 52.3439) (end 160.6439 52.3439) (width 0.2) (layer "F.Cu") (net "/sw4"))
 (segment (start 177.01 44.4) (end 178.81 46.2) (width 0.2) (layer "F.Cu") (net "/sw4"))
 (segment (start 181.6725 52.6275) (end 178.6275 52.6275) (width 0.2) (layer "F.Cu") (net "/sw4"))
 (segment (start 169.312412 50.387588) (end 167.3561 52.3439) (width 0.2) (layer "F.Cu") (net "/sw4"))
 (segment (start 194.46 47.46) (end 194.4 47.4) (width 0.2) (layer "F.Cu") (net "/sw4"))
 (segment (start 178.6275 52.6275) (end 178.1 52.1) (width 0.2) (layer "F.Cu") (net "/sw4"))
 (segment (start 196.19 47.46) (end 194.46 47.46) (width 0.2) (layer "F.Cu") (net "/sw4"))
 (segment (start 186.6 47.7) (end 183.3439 50.9561) (width 0.2) (layer "F.Cu") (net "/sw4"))
 (segment (start 181.9561 52.3439) (end 181.6725 52.6275) (width 0.2) (layer "F.Cu") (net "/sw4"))
 (segment (start 186.6 47) (end 186.6 47.7) (width 0.2) (layer "F.Cu") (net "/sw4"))
 (via (at 170.1 48.6) (size 0.6) (drill 0.3) (layers "F.Cu" "B.Cu") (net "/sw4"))
 (via (at 194.4 47.4) (size 0.6) (drill 0.3) (layers "F.Cu" "B.Cu") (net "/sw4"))
 (via (at 178.9 46.2) (size 0.6) (drill 0.3) (layers "F.Cu" "B.Cu") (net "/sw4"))
 (via (at 186.6 47) (size 0.6) (drill 0.3) (layers "F.Cu" "B.Cu") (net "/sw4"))
 (via (at 178.1 49.6) (size 0.6) (drill 0.3) (layers "F.Cu" "B.Cu") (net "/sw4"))
 (segment (start 178.8 47.865255) (end 178.8 46.3) (width 0.2) (layer "B.Cu") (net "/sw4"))
 (segment (start 176.599745 48.885) (end 177.780255 48.885) (width 0.2) (layer "B.Cu") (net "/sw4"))
 (segment (start 176.214745 48.5) (end 176.599745 48.885) (width 0.2) (layer "B.Cu") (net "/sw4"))
 (segment (start 178.8 46.3) (end 178.9 46.2) (width 0.2) (layer "B.Cu") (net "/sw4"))
 (segment (start 177.780255 48.885) (end 178.8 47.865255) (width 0.2) (layer "B.Cu") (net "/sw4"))
 (segment (start 170.1 48.6) (end 170.2 48.5) (width 0.2) (layer "B.Cu") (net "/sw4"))
 (segment (start 178.1 49.6) (end 178.1 49.204745) (width 0.2) (layer "B.Cu") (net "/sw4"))
 (segment (start 187 47.4) (end 186.6 47) (width 0.2) (layer "B.Cu") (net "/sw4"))
 (segment (start 170.2 48.5) (end 176.214745 48.5) (width 0.2) (layer "B.Cu") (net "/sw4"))
 (segment (start 178.1 49.204745) (end 177.780255 48.885) (width 0.2) (layer "B.Cu") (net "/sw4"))
 (segment (start 194.4 47.4) (end 187 47.4) (width 0.2) (layer "B.Cu") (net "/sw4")))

